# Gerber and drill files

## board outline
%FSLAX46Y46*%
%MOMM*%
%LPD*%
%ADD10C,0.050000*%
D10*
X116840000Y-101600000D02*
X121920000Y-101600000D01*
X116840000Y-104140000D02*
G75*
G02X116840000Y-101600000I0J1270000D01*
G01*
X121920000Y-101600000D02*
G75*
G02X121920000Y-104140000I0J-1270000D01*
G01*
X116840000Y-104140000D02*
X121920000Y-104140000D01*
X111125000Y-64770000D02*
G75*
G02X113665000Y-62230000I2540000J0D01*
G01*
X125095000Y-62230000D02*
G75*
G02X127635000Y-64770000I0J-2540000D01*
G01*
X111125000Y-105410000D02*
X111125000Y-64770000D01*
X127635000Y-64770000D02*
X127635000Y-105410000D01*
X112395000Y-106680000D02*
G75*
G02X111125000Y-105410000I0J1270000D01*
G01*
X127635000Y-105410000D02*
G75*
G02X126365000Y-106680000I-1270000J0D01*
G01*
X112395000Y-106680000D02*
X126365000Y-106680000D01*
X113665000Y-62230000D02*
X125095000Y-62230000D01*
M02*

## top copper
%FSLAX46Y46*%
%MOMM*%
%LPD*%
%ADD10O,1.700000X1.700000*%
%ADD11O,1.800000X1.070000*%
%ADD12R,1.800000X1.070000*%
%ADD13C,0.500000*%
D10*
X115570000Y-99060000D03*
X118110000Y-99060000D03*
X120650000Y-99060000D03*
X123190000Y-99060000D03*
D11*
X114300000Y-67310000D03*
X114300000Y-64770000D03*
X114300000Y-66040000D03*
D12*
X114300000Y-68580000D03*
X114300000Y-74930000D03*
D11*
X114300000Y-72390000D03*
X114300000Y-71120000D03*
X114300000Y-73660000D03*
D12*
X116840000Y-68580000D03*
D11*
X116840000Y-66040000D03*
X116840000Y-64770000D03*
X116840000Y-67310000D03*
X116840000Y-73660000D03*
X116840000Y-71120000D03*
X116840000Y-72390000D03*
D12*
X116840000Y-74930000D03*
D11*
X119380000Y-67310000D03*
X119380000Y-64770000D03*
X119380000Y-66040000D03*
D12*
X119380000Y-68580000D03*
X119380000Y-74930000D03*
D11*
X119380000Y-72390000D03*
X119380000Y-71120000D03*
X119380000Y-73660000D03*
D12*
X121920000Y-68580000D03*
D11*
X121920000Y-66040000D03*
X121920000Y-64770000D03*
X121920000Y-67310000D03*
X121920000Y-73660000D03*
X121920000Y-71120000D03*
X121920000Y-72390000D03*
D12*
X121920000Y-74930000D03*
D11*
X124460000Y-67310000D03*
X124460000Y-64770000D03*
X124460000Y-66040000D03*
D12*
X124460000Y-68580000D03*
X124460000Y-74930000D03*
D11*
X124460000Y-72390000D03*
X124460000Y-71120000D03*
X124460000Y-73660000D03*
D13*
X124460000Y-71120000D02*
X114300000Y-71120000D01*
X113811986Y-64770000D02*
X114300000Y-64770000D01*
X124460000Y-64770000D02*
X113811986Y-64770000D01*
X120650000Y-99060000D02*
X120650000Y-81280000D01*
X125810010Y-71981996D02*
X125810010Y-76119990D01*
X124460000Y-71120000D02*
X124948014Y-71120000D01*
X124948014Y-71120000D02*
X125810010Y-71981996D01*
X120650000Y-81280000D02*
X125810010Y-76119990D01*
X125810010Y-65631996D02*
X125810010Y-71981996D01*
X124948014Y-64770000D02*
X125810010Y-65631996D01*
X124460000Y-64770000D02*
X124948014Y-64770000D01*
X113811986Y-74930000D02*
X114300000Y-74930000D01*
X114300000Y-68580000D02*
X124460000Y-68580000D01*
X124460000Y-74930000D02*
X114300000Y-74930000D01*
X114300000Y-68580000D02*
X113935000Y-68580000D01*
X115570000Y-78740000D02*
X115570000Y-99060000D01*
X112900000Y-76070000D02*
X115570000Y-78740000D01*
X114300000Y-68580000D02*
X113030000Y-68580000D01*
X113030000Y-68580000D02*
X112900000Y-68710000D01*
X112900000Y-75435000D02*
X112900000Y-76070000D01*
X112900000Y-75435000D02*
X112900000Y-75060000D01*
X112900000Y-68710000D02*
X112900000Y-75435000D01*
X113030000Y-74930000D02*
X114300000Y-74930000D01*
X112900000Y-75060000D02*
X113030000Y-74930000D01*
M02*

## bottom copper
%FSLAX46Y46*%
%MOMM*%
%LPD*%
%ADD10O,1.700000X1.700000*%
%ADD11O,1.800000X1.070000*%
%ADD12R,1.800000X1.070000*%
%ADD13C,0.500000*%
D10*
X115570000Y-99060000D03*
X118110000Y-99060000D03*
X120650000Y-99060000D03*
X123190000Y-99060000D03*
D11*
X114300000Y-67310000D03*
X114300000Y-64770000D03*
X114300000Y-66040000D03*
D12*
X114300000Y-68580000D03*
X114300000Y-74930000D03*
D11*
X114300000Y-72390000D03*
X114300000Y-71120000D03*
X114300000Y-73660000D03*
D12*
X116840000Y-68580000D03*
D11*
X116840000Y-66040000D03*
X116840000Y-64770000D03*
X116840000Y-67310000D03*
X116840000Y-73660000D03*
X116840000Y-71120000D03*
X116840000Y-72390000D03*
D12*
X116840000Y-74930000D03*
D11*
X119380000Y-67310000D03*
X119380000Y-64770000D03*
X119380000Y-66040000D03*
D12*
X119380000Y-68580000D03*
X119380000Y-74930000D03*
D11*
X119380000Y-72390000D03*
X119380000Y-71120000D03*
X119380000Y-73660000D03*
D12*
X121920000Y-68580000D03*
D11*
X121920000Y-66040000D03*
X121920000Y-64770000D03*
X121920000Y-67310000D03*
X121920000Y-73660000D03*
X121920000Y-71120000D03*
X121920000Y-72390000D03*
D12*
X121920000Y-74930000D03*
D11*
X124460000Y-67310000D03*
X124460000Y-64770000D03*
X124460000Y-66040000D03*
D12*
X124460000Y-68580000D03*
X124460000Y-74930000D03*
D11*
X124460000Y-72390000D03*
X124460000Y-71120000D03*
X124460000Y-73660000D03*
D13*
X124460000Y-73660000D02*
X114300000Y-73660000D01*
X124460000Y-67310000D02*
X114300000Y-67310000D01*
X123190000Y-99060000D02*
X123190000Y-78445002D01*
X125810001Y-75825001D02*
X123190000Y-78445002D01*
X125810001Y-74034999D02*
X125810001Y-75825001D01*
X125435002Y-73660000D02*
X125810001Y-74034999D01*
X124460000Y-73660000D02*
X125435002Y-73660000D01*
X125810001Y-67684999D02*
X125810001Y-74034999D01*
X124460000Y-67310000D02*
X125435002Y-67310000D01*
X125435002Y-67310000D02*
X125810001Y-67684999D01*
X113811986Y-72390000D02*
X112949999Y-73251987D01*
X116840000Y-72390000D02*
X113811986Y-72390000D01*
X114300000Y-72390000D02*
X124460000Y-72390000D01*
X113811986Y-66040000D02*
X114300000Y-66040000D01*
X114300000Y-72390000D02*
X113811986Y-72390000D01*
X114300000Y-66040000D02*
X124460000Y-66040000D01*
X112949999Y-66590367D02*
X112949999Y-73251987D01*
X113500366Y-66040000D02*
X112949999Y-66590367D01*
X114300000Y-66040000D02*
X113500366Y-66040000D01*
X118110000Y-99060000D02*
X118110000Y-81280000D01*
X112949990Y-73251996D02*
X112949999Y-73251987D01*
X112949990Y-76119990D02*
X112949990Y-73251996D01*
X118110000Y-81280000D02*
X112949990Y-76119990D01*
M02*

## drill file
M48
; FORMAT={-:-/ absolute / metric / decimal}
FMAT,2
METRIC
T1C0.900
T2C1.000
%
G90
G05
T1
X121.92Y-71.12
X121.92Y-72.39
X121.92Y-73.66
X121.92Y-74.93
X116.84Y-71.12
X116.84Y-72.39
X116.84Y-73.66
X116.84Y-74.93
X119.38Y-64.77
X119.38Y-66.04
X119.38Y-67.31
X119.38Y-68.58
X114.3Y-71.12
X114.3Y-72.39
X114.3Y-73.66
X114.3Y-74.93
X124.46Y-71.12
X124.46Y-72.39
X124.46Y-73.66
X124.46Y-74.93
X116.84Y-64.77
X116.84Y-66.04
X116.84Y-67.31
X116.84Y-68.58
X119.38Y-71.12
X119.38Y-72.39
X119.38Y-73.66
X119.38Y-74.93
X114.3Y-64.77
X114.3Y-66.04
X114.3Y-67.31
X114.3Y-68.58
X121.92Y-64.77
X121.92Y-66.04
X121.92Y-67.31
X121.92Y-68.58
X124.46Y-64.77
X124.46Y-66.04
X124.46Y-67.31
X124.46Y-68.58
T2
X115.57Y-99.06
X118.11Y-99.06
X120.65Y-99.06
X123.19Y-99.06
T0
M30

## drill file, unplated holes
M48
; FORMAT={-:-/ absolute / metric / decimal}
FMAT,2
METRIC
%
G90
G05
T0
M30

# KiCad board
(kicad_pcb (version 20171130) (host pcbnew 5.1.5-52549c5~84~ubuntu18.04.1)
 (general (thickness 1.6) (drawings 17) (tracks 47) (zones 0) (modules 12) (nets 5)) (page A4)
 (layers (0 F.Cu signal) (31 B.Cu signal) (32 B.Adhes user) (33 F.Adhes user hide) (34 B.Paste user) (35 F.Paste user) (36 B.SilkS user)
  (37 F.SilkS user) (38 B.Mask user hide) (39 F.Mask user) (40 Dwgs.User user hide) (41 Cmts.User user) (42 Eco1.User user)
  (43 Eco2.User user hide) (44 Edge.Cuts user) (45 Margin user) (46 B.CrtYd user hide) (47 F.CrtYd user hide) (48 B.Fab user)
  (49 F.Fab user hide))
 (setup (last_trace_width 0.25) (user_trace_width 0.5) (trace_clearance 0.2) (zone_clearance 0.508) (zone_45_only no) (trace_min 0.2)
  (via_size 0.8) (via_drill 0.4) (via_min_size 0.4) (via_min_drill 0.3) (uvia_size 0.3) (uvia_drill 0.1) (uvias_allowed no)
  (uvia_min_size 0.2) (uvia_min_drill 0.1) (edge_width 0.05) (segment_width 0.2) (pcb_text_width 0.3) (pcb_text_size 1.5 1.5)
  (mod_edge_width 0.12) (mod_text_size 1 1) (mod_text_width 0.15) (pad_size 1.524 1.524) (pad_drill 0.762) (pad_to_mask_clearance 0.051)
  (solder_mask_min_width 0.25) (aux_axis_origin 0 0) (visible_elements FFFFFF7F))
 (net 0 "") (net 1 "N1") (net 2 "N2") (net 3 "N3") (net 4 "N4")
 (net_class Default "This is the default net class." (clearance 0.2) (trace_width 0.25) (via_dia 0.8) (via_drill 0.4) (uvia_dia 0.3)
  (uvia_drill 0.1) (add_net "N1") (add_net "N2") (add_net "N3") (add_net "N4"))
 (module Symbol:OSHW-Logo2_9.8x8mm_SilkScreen (layer F.Cu) (at 119.38 87.63)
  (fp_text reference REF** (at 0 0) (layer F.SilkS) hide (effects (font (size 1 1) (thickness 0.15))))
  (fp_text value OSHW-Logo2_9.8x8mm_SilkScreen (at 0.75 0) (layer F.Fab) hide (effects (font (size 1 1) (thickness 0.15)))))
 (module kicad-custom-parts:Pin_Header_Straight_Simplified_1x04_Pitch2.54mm (layer F.Cu) (at 115.57 99.06 90)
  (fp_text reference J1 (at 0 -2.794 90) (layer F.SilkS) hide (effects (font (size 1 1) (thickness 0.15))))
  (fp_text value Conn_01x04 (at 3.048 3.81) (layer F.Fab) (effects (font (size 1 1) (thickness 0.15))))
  (pad 1 thru_hole oval (at 0 0 90) (size 1.7 1.7) (drill 1) (layers *.Cu *.Mask) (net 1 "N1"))
  (pad 2 thru_hole oval (at 0 2.54 90) (size 1.7 1.7) (drill 1) (layers *.Cu *.Mask) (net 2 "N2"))
  (pad 3 thru_hole oval (at 0 5.08 90) (size 1.7 1.7) (drill 1) (layers *.Cu *.Mask) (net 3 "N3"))
  (pad 4 thru_hole oval (at 0 7.62 90) (size 1.7 1.7) (drill 1) (layers *.Cu *.Mask) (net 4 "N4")))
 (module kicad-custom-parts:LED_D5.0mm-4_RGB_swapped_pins (layer F.Cu) (at 114.3 68.58 90)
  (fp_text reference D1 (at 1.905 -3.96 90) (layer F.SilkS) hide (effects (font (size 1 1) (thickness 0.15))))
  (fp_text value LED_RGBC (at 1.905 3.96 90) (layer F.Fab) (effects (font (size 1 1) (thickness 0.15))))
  (pad 4 thru_hole oval (at 1.27 0 90) (size 1.07 1.8) (drill 0.9) (layers *.Cu *.Mask) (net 4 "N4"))
  (pad 3 thru_hole oval (at 3.81 0 90) (size 1.07 1.8) (drill 0.9) (layers *.Cu *.Mask) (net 3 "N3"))
  (pad 2 thru_hole oval (at 2.54 0 90) (size 1.07 1.8) (drill 0.9) (layers *.Cu *.Mask) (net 2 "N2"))
  (pad 1 thru_hole rect (at 0 0 90) (size 1.07 1.8) (drill 0.9) (layers *.Cu *.Mask) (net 1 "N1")))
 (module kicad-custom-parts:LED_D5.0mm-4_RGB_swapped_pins (layer F.Cu) (at 114.3 74.93 90)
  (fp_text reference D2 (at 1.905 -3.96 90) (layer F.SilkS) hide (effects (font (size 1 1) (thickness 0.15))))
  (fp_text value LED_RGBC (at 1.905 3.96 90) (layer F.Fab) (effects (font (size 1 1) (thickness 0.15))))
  (pad 1 thru_hole rect (at 0 0 90) (size 1.07 1.8) (drill 0.9) (layers *.Cu *.Mask) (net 1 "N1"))
  (pad 2 thru_hole oval (at 2.54 0 90) (size 1.07 1.8) (drill 0.9) (layers *.Cu *.Mask) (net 2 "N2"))
  (pad 3 thru_hole oval (at 3.81 0 90) (size 1.07 1.8) (drill 0.9) (layers *.Cu *.Mask) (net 3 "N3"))
  (pad 4 thru_hole oval (at 1.27 0 90) (size 1.07 1.8) (drill 0.9) (layers *.Cu *.Mask) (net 4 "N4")))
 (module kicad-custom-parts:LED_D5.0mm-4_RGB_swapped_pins (layer F.Cu) (at 116.84 68.58 90)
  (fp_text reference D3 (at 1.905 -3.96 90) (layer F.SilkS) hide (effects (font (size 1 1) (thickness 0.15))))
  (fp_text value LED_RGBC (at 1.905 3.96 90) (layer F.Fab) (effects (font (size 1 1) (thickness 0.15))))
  (pad 1 thru_hole rect (at 0 0 90) (size 1.07 1.8) (drill 0.9) (layers *.Cu *.Mask) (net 1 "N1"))
  (pad 2 thru_hole oval (at 2.54 0 90) (size 1.07 1.8) (drill 0.9) (layers *.Cu *.Mask) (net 2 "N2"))
  (pad 3 thru_hole oval (at 3.81 0 90) (size 1.07 1.8) (drill 0.9) (layers *.Cu *.Mask) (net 3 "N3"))
  (pad 4 thru_hole oval (at 1.27 0 90) (size 1.07 1.8) (drill 0.9) (layers *.Cu *.Mask) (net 4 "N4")))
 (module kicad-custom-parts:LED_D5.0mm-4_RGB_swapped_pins (layer F.Cu) (at 116.84 74.93 90)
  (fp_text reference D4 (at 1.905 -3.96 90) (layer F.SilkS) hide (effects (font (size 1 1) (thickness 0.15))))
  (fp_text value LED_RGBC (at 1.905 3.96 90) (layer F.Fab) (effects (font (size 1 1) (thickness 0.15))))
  (pad 4 thru_hole oval (at 1.27 0 90) (size 1.07 1.8) (drill 0.9) (layers *.Cu *.Mask) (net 4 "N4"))
  (pad 3 thru_hole oval (at 3.81 0 90) (size 1.07 1.8) (drill 0.9) (layers *.Cu *.Mask) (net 3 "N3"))
  (pad 2 thru_hole oval (at 2.54 0 90) (size 1.07 1.8) (drill 0.9) (layers *.Cu *.Mask) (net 2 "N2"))
  (pad 1 thru_hole rect (at 0 0 90) (size 1.07 1.8) (drill 0.9) (layers *.Cu *.Mask) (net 1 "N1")))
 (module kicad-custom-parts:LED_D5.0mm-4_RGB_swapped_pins (layer F.Cu) (at 119.38 68.58 90)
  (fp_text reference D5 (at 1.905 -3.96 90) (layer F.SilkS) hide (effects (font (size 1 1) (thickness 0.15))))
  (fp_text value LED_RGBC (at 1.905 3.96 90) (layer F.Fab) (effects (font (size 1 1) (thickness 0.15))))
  (pad 4 thru_hole oval (at 1.27 0 90) (size 1.07 1.8) (drill 0.9) (layers *.Cu *.Mask) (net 4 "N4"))
  (pad 3 thru_hole oval (at 3.81 0 90) (size 1.07 1.8) (drill 0.9) (layers *.Cu *.Mask) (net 3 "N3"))
  (pad 2 thru_hole oval (at 2.54 0 90) (size 1.07 1.8) (drill 0.9) (layers *.Cu *.Mask) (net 2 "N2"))
  (pad 1 thru_hole rect (at 0 0 90) (size 1.07 1.8) (drill 0.9) (layers *.Cu *.Mask) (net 1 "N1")))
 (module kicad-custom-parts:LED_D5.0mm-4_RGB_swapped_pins (layer F.Cu) (at 119.38 74.93 90)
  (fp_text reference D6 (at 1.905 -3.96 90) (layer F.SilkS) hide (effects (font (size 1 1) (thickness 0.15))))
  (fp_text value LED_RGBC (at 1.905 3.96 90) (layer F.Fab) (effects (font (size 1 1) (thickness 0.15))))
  (pad 1 thru_hole rect (at 0 0 90) (size 1.07 1.8) (drill 0.9) (layers *.Cu *.Mask) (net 1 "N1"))
  (pad 2 thru_hole oval (at 2.54 0 90) (size 1.07 1.8) (drill 0.9) (layers *.Cu *.Mask) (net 2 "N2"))
  (pad 3 thru_hole oval (at 3.81 0 90) (size 1.07 1.8) (drill 0.9) (layers *.Cu *.Mask) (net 3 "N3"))
  (pad 4 thru_hole oval (at 1.27 0 90) (size 1.07 1.8) (drill 0.9) (layers *.Cu *.Mask) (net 4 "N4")))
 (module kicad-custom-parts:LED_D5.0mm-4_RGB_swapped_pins (layer F.Cu) (at 121.92 68.58 90)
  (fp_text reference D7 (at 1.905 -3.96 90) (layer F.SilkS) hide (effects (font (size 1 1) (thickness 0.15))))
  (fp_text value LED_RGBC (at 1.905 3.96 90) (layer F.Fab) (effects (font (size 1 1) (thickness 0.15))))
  (pad 1 thru_hole rect (at 0 0 90) (size 1.07 1.8) (drill 0.9) (layers *.Cu *.Mask) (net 1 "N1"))
  (pad 2 thru_hole oval (at 2.54 0 90) (size 1.07 1.8) (drill 0.9) (layers *.Cu *.Mask) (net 2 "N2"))
  (pad 3 thru_hole oval (at 3.81 0 90) (size 1.07 1.8) (drill 0.9) (layers *.Cu *.Mask) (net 3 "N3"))
  (pad 4 thru_hole oval (at 1.27 0 90) (size 1.07 1.8) (drill 0.9) (layers *.Cu *.Mask) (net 4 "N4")))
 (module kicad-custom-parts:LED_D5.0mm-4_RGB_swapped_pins (layer F.Cu) (at 121.92 74.93 90)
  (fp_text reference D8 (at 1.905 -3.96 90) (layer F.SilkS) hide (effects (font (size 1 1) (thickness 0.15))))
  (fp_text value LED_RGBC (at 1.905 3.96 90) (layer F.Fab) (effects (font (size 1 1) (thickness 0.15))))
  (pad 4 thru_hole oval (at 1.27 0 90) (size 1.07 1.8) (drill 0.9) (layers *.Cu *.Mask) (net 4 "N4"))
  (pad 3 thru_hole oval (at 3.81 0 90) (size 1.07 1.8) (drill 0.9) (layers *.Cu *.Mask) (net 3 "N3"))
  (pad 2 thru_hole oval (at 2.54 0 90) (size 1.07 1.8) (drill 0.9) (layers *.Cu *.Mask) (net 2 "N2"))
  (pad 1 thru_hole rect (at 0 0 90) (size 1.07 1.8) (drill 0.9) (layers *.Cu *.Mask) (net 1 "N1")))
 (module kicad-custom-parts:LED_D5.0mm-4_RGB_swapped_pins (layer F.Cu) (at 124.46 68.58 90)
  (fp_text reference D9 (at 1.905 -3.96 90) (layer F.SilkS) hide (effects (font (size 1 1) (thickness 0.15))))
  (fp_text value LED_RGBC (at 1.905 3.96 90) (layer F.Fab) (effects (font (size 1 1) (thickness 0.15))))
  (pad 4 thru_hole oval (at 1.27 0 90) (size 1.07 1.8) (drill 0.9) (layers *.Cu *.Mask) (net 4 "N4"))
  (pad 3 thru_hole oval (at 3.81 0 90) (size 1.07 1.8) (drill 0.9) (layers *.Cu *.Mask) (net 3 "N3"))
  (pad 2 thru_hole oval (at 2.54 0 90) (size 1.07 1.8) (drill 0.9) (layers *.Cu *.Mask) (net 2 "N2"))
  (pad 1 thru_hole rect (at 0 0 90) (size 1.07 1.8) (drill 0.9) (layers *.Cu *.Mask) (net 1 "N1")))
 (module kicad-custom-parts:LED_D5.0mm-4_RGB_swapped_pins (layer F.Cu) (at 124.46 74.93 90)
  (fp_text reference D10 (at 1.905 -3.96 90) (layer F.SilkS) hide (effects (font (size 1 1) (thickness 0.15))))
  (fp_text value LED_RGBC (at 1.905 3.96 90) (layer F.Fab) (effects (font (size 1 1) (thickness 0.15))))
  (pad 1 thru_hole rect (at 0 0 90) (size 1.07 1.8) (drill 0.9) (layers *.Cu *.Mask) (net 1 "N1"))
  (pad 2 thru_hole oval (at 2.54 0 90) (size 1.07 1.8) (drill 0.9) (layers *.Cu *.Mask) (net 2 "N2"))
  (pad 3 thru_hole oval (at 3.81 0 90) (size 1.07 1.8) (drill 0.9) (layers *.Cu *.Mask) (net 3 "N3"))
  (pad 4 thru_hole oval (at 1.27 0 90) (size 1.07 1.8) (drill 0.9) (layers *.Cu *.Mask) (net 4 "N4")))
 (gr_line (start 116.84 101.6) (end 121.92 101.6) (layer Edge.Cuts) (width 0.05))
 (gr_arc (start 116.84 102.87) (end 116.84 101.6) (angle -180) (layer Edge.Cuts) (width 0.05))
 (gr_arc (start 121.92 102.87) (end 121.92 104.14) (angle -180) (layer Edge.Cuts) (width 0.05))
 (gr_line (start 116.84 104.14) (end 121.92 104.14) (layer Edge.Cuts) (width 0.05))
 (gr_arc (start 113.665 64.77) (end 113.665 62.23) (angle -90) (layer Edge.Cuts) (width 0.05))
 (gr_arc (start 125.095 64.77) (end 127.635 64.77) (angle -90) (layer Edge.Cuts) (width 0.05))
 (gr_line (start 111.125 105.41) (end 111.125 64.77) (layer Edge.Cuts) (width 0.05))
 (gr_line (start 127.635 64.77) (end 127.635 105.41) (layer Edge.Cuts) (width 0.05))
 (gr_arc (start 112.395 105.41) (end 111.125 105.41) (angle -90) (layer Edge.Cuts) (width 0.05))
 (gr_arc (start 126.365 105.41) (end 126.365 106.68) (angle -90) (layer Edge.Cuts) (width 0.05))
 (gr_line (start 112.395 106.68) (end 126.365 106.68) (layer Edge.Cuts) (width 0.05))
 (gr_line (start 113.665 62.23) (end 125.095 62.23) (layer Edge.Cuts) (width 0.05))
 (segment (start 124.46 73.66) (end 114.3 73.66) (width 0.5) (layer B.Cu) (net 4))
 (segment (start 124.46 67.31) (end 114.3 67.31) (width 0.5) (layer B.Cu) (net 4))
 (segment (start 123.19 99.06) (end 123.19 78.445002) (width 0.5) (layer B.Cu) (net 4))
 (segment (start 125.810001 75.825001) (end 123.19 78.445002) (width 0.5) (layer B.Cu) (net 4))
 (segment (start 125.810001 74.034999) (end 125.810001 75.825001) (width 0.5) (layer B.Cu) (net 4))
 (segment (start 125.435002 73.66) (end 125.810001 74.034999) (width 0.5) (layer B.Cu) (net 4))
 (segment (start 124.46 73.66) (end 125.435002 73.66) (width 0.5) (layer B.Cu) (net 4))
 (segment (start 125.810001 67.684999) (end 125.810001 74.034999) (width 0.5) (layer B.Cu) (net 4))
 (segment (start 124.46 67.31) (end 125.435002 67.31) (width 0.5) (layer B.Cu) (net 4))
 (segment (start 125.435002 67.31) (end 125.810001 67.684999) (width 0.5) (layer B.Cu) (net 4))
 (segment (start 124.46 71.12) (end 114.3 71.12) (width 0.5) (layer F.Cu) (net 3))
 (segment (start 113.811986 64.77) (end 114.3 64.77) (width 0.5) (layer F.Cu) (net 3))
 (segment (start 124.46 64.77) (end 113.811986 64.77) (width 0.5) (layer F.Cu) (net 3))
 (segment (start 120.65 99.06) (end 120.65 81.28) (width 0.5) (layer F.Cu) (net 3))
 (segment (start 125.81001 71.981996) (end 125.81001 76.11999) (width 0.5) (layer F.Cu) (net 3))
 (segment (start 124.46 71.12) (end 124.948014 71.12) (width 0.5) (layer F.Cu) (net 3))
 (segment (start 124.948014 71.12) (end 125.81001 71.981996) (width 0.5) (layer F.Cu) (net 3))
 (segment (start 120.65 81.28) (end 125.81001 76.11999) (width 0.5) (layer F.Cu) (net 3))
 (segment (start 125.81001 65.631996) (end 125.81001 71.981996) (width 0.5) (layer F.Cu) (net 3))
 (segment (start 124.948014 64.77) (end 125.81001 65.631996) (width 0.5) (layer F.Cu) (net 3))
 (segment (start 124.46 64.77) (end 124.948014 64.77) (width 0.5) (layer F.Cu) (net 3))
 (segment (start 113.811986 72.39) (end 112.949999 73.251987) (width 0.5) (layer B.Cu) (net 2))
 (segment (start 116.84 72.39) (end 113.811986 72.39) (width 0.5) (layer B.Cu) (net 2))
 (segment (start 114.3 72.39) (end 124.46 72.39) (width 0.5) (layer B.Cu) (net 2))
 (segment (start 113.811986 66.04) (end 114.3 66.04) (width 0.5) (layer B.Cu) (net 2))
 (segment (start 114.3 72.39) (end 113.811986 72.39) (width 0.5) (layer B.Cu) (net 2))
 (segment (start 114.3 66.04) (end 124.46 66.04) (width 0.5) (layer B.Cu) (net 2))
 (segment (start 112.949999 66.590367) (end 112.949999 73.251987) (width 0.5) (layer B.Cu) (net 2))
 (segment (start 113.500366 66.04) (end 112.949999 66.590367) (width 0.5) (layer B.Cu) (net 2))
 (segment (start 114.3 66.04) (end 113.500366 66.04) (width 0.5) (layer B.Cu) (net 2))
 (segment (start 118.11 99.06) (end 118.11 81.28) (width 0.5) (layer B.Cu) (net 2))
 (segment (start 112.94999 73.251996) (end 112.949999 73.251987) (width 0.5) (layer B.Cu) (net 2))
 (segment (start 112.94999 76.11999) (end 112.94999 73.251996) (width 0.5) (layer B.Cu) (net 2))
 (segment (start 118.11 81.28) (end 112.94999 76.11999) (width 0.5) (layer B.Cu) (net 2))
 (segment (start 113.811986 74.93) (end 114.3 74.93) (width 0.5) (layer F.Cu) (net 1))
 (segment (start 114.3 68.58) (end 124.46 68.58) (width 0.5) (layer F.Cu) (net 1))
 (segment (start 124.46 74.93) (end 114.3 74.93) (width 0.5) (layer F.Cu) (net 1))
 (segment (start 114.3 68.58) (end 113.935 68.58) (width 0.5) (layer F.Cu) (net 1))
 (segment (start 115.57 78.74) (end 115.57 99.06) (width 0.5) (layer F.Cu) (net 1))
 (segment (start 112.9 76.07) (end 115.57 78.74) (width 0.5) (layer F.Cu) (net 1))
 (segment (start 114.3 68.58) (end 113.03 68.58) (width 0.5) (layer F.Cu) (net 1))
 (segment (start 113.03 68.58) (end 112.9 68.71) (width 0.5) (layer F.Cu) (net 1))
 (segment (start 112.9 75.435) (end 112.9 76.07) (width 0.5) (layer F.Cu) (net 1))
 (segment (start 112.9 75.435) (end 112.9 75.06) (width 0.5) (layer F.Cu) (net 1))
 (segment (start 112.9 68.71) (end 112.9 75.435) (width 0.5) (layer F.Cu) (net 1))
 (segment (start 113.03 74.93) (end 114.3 74.93) (width 0.5) (layer F.Cu) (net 1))
 (segment (start 112.9 75.06) (end 113.03 74.93) (width 0.5) (layer F.Cu) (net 1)))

